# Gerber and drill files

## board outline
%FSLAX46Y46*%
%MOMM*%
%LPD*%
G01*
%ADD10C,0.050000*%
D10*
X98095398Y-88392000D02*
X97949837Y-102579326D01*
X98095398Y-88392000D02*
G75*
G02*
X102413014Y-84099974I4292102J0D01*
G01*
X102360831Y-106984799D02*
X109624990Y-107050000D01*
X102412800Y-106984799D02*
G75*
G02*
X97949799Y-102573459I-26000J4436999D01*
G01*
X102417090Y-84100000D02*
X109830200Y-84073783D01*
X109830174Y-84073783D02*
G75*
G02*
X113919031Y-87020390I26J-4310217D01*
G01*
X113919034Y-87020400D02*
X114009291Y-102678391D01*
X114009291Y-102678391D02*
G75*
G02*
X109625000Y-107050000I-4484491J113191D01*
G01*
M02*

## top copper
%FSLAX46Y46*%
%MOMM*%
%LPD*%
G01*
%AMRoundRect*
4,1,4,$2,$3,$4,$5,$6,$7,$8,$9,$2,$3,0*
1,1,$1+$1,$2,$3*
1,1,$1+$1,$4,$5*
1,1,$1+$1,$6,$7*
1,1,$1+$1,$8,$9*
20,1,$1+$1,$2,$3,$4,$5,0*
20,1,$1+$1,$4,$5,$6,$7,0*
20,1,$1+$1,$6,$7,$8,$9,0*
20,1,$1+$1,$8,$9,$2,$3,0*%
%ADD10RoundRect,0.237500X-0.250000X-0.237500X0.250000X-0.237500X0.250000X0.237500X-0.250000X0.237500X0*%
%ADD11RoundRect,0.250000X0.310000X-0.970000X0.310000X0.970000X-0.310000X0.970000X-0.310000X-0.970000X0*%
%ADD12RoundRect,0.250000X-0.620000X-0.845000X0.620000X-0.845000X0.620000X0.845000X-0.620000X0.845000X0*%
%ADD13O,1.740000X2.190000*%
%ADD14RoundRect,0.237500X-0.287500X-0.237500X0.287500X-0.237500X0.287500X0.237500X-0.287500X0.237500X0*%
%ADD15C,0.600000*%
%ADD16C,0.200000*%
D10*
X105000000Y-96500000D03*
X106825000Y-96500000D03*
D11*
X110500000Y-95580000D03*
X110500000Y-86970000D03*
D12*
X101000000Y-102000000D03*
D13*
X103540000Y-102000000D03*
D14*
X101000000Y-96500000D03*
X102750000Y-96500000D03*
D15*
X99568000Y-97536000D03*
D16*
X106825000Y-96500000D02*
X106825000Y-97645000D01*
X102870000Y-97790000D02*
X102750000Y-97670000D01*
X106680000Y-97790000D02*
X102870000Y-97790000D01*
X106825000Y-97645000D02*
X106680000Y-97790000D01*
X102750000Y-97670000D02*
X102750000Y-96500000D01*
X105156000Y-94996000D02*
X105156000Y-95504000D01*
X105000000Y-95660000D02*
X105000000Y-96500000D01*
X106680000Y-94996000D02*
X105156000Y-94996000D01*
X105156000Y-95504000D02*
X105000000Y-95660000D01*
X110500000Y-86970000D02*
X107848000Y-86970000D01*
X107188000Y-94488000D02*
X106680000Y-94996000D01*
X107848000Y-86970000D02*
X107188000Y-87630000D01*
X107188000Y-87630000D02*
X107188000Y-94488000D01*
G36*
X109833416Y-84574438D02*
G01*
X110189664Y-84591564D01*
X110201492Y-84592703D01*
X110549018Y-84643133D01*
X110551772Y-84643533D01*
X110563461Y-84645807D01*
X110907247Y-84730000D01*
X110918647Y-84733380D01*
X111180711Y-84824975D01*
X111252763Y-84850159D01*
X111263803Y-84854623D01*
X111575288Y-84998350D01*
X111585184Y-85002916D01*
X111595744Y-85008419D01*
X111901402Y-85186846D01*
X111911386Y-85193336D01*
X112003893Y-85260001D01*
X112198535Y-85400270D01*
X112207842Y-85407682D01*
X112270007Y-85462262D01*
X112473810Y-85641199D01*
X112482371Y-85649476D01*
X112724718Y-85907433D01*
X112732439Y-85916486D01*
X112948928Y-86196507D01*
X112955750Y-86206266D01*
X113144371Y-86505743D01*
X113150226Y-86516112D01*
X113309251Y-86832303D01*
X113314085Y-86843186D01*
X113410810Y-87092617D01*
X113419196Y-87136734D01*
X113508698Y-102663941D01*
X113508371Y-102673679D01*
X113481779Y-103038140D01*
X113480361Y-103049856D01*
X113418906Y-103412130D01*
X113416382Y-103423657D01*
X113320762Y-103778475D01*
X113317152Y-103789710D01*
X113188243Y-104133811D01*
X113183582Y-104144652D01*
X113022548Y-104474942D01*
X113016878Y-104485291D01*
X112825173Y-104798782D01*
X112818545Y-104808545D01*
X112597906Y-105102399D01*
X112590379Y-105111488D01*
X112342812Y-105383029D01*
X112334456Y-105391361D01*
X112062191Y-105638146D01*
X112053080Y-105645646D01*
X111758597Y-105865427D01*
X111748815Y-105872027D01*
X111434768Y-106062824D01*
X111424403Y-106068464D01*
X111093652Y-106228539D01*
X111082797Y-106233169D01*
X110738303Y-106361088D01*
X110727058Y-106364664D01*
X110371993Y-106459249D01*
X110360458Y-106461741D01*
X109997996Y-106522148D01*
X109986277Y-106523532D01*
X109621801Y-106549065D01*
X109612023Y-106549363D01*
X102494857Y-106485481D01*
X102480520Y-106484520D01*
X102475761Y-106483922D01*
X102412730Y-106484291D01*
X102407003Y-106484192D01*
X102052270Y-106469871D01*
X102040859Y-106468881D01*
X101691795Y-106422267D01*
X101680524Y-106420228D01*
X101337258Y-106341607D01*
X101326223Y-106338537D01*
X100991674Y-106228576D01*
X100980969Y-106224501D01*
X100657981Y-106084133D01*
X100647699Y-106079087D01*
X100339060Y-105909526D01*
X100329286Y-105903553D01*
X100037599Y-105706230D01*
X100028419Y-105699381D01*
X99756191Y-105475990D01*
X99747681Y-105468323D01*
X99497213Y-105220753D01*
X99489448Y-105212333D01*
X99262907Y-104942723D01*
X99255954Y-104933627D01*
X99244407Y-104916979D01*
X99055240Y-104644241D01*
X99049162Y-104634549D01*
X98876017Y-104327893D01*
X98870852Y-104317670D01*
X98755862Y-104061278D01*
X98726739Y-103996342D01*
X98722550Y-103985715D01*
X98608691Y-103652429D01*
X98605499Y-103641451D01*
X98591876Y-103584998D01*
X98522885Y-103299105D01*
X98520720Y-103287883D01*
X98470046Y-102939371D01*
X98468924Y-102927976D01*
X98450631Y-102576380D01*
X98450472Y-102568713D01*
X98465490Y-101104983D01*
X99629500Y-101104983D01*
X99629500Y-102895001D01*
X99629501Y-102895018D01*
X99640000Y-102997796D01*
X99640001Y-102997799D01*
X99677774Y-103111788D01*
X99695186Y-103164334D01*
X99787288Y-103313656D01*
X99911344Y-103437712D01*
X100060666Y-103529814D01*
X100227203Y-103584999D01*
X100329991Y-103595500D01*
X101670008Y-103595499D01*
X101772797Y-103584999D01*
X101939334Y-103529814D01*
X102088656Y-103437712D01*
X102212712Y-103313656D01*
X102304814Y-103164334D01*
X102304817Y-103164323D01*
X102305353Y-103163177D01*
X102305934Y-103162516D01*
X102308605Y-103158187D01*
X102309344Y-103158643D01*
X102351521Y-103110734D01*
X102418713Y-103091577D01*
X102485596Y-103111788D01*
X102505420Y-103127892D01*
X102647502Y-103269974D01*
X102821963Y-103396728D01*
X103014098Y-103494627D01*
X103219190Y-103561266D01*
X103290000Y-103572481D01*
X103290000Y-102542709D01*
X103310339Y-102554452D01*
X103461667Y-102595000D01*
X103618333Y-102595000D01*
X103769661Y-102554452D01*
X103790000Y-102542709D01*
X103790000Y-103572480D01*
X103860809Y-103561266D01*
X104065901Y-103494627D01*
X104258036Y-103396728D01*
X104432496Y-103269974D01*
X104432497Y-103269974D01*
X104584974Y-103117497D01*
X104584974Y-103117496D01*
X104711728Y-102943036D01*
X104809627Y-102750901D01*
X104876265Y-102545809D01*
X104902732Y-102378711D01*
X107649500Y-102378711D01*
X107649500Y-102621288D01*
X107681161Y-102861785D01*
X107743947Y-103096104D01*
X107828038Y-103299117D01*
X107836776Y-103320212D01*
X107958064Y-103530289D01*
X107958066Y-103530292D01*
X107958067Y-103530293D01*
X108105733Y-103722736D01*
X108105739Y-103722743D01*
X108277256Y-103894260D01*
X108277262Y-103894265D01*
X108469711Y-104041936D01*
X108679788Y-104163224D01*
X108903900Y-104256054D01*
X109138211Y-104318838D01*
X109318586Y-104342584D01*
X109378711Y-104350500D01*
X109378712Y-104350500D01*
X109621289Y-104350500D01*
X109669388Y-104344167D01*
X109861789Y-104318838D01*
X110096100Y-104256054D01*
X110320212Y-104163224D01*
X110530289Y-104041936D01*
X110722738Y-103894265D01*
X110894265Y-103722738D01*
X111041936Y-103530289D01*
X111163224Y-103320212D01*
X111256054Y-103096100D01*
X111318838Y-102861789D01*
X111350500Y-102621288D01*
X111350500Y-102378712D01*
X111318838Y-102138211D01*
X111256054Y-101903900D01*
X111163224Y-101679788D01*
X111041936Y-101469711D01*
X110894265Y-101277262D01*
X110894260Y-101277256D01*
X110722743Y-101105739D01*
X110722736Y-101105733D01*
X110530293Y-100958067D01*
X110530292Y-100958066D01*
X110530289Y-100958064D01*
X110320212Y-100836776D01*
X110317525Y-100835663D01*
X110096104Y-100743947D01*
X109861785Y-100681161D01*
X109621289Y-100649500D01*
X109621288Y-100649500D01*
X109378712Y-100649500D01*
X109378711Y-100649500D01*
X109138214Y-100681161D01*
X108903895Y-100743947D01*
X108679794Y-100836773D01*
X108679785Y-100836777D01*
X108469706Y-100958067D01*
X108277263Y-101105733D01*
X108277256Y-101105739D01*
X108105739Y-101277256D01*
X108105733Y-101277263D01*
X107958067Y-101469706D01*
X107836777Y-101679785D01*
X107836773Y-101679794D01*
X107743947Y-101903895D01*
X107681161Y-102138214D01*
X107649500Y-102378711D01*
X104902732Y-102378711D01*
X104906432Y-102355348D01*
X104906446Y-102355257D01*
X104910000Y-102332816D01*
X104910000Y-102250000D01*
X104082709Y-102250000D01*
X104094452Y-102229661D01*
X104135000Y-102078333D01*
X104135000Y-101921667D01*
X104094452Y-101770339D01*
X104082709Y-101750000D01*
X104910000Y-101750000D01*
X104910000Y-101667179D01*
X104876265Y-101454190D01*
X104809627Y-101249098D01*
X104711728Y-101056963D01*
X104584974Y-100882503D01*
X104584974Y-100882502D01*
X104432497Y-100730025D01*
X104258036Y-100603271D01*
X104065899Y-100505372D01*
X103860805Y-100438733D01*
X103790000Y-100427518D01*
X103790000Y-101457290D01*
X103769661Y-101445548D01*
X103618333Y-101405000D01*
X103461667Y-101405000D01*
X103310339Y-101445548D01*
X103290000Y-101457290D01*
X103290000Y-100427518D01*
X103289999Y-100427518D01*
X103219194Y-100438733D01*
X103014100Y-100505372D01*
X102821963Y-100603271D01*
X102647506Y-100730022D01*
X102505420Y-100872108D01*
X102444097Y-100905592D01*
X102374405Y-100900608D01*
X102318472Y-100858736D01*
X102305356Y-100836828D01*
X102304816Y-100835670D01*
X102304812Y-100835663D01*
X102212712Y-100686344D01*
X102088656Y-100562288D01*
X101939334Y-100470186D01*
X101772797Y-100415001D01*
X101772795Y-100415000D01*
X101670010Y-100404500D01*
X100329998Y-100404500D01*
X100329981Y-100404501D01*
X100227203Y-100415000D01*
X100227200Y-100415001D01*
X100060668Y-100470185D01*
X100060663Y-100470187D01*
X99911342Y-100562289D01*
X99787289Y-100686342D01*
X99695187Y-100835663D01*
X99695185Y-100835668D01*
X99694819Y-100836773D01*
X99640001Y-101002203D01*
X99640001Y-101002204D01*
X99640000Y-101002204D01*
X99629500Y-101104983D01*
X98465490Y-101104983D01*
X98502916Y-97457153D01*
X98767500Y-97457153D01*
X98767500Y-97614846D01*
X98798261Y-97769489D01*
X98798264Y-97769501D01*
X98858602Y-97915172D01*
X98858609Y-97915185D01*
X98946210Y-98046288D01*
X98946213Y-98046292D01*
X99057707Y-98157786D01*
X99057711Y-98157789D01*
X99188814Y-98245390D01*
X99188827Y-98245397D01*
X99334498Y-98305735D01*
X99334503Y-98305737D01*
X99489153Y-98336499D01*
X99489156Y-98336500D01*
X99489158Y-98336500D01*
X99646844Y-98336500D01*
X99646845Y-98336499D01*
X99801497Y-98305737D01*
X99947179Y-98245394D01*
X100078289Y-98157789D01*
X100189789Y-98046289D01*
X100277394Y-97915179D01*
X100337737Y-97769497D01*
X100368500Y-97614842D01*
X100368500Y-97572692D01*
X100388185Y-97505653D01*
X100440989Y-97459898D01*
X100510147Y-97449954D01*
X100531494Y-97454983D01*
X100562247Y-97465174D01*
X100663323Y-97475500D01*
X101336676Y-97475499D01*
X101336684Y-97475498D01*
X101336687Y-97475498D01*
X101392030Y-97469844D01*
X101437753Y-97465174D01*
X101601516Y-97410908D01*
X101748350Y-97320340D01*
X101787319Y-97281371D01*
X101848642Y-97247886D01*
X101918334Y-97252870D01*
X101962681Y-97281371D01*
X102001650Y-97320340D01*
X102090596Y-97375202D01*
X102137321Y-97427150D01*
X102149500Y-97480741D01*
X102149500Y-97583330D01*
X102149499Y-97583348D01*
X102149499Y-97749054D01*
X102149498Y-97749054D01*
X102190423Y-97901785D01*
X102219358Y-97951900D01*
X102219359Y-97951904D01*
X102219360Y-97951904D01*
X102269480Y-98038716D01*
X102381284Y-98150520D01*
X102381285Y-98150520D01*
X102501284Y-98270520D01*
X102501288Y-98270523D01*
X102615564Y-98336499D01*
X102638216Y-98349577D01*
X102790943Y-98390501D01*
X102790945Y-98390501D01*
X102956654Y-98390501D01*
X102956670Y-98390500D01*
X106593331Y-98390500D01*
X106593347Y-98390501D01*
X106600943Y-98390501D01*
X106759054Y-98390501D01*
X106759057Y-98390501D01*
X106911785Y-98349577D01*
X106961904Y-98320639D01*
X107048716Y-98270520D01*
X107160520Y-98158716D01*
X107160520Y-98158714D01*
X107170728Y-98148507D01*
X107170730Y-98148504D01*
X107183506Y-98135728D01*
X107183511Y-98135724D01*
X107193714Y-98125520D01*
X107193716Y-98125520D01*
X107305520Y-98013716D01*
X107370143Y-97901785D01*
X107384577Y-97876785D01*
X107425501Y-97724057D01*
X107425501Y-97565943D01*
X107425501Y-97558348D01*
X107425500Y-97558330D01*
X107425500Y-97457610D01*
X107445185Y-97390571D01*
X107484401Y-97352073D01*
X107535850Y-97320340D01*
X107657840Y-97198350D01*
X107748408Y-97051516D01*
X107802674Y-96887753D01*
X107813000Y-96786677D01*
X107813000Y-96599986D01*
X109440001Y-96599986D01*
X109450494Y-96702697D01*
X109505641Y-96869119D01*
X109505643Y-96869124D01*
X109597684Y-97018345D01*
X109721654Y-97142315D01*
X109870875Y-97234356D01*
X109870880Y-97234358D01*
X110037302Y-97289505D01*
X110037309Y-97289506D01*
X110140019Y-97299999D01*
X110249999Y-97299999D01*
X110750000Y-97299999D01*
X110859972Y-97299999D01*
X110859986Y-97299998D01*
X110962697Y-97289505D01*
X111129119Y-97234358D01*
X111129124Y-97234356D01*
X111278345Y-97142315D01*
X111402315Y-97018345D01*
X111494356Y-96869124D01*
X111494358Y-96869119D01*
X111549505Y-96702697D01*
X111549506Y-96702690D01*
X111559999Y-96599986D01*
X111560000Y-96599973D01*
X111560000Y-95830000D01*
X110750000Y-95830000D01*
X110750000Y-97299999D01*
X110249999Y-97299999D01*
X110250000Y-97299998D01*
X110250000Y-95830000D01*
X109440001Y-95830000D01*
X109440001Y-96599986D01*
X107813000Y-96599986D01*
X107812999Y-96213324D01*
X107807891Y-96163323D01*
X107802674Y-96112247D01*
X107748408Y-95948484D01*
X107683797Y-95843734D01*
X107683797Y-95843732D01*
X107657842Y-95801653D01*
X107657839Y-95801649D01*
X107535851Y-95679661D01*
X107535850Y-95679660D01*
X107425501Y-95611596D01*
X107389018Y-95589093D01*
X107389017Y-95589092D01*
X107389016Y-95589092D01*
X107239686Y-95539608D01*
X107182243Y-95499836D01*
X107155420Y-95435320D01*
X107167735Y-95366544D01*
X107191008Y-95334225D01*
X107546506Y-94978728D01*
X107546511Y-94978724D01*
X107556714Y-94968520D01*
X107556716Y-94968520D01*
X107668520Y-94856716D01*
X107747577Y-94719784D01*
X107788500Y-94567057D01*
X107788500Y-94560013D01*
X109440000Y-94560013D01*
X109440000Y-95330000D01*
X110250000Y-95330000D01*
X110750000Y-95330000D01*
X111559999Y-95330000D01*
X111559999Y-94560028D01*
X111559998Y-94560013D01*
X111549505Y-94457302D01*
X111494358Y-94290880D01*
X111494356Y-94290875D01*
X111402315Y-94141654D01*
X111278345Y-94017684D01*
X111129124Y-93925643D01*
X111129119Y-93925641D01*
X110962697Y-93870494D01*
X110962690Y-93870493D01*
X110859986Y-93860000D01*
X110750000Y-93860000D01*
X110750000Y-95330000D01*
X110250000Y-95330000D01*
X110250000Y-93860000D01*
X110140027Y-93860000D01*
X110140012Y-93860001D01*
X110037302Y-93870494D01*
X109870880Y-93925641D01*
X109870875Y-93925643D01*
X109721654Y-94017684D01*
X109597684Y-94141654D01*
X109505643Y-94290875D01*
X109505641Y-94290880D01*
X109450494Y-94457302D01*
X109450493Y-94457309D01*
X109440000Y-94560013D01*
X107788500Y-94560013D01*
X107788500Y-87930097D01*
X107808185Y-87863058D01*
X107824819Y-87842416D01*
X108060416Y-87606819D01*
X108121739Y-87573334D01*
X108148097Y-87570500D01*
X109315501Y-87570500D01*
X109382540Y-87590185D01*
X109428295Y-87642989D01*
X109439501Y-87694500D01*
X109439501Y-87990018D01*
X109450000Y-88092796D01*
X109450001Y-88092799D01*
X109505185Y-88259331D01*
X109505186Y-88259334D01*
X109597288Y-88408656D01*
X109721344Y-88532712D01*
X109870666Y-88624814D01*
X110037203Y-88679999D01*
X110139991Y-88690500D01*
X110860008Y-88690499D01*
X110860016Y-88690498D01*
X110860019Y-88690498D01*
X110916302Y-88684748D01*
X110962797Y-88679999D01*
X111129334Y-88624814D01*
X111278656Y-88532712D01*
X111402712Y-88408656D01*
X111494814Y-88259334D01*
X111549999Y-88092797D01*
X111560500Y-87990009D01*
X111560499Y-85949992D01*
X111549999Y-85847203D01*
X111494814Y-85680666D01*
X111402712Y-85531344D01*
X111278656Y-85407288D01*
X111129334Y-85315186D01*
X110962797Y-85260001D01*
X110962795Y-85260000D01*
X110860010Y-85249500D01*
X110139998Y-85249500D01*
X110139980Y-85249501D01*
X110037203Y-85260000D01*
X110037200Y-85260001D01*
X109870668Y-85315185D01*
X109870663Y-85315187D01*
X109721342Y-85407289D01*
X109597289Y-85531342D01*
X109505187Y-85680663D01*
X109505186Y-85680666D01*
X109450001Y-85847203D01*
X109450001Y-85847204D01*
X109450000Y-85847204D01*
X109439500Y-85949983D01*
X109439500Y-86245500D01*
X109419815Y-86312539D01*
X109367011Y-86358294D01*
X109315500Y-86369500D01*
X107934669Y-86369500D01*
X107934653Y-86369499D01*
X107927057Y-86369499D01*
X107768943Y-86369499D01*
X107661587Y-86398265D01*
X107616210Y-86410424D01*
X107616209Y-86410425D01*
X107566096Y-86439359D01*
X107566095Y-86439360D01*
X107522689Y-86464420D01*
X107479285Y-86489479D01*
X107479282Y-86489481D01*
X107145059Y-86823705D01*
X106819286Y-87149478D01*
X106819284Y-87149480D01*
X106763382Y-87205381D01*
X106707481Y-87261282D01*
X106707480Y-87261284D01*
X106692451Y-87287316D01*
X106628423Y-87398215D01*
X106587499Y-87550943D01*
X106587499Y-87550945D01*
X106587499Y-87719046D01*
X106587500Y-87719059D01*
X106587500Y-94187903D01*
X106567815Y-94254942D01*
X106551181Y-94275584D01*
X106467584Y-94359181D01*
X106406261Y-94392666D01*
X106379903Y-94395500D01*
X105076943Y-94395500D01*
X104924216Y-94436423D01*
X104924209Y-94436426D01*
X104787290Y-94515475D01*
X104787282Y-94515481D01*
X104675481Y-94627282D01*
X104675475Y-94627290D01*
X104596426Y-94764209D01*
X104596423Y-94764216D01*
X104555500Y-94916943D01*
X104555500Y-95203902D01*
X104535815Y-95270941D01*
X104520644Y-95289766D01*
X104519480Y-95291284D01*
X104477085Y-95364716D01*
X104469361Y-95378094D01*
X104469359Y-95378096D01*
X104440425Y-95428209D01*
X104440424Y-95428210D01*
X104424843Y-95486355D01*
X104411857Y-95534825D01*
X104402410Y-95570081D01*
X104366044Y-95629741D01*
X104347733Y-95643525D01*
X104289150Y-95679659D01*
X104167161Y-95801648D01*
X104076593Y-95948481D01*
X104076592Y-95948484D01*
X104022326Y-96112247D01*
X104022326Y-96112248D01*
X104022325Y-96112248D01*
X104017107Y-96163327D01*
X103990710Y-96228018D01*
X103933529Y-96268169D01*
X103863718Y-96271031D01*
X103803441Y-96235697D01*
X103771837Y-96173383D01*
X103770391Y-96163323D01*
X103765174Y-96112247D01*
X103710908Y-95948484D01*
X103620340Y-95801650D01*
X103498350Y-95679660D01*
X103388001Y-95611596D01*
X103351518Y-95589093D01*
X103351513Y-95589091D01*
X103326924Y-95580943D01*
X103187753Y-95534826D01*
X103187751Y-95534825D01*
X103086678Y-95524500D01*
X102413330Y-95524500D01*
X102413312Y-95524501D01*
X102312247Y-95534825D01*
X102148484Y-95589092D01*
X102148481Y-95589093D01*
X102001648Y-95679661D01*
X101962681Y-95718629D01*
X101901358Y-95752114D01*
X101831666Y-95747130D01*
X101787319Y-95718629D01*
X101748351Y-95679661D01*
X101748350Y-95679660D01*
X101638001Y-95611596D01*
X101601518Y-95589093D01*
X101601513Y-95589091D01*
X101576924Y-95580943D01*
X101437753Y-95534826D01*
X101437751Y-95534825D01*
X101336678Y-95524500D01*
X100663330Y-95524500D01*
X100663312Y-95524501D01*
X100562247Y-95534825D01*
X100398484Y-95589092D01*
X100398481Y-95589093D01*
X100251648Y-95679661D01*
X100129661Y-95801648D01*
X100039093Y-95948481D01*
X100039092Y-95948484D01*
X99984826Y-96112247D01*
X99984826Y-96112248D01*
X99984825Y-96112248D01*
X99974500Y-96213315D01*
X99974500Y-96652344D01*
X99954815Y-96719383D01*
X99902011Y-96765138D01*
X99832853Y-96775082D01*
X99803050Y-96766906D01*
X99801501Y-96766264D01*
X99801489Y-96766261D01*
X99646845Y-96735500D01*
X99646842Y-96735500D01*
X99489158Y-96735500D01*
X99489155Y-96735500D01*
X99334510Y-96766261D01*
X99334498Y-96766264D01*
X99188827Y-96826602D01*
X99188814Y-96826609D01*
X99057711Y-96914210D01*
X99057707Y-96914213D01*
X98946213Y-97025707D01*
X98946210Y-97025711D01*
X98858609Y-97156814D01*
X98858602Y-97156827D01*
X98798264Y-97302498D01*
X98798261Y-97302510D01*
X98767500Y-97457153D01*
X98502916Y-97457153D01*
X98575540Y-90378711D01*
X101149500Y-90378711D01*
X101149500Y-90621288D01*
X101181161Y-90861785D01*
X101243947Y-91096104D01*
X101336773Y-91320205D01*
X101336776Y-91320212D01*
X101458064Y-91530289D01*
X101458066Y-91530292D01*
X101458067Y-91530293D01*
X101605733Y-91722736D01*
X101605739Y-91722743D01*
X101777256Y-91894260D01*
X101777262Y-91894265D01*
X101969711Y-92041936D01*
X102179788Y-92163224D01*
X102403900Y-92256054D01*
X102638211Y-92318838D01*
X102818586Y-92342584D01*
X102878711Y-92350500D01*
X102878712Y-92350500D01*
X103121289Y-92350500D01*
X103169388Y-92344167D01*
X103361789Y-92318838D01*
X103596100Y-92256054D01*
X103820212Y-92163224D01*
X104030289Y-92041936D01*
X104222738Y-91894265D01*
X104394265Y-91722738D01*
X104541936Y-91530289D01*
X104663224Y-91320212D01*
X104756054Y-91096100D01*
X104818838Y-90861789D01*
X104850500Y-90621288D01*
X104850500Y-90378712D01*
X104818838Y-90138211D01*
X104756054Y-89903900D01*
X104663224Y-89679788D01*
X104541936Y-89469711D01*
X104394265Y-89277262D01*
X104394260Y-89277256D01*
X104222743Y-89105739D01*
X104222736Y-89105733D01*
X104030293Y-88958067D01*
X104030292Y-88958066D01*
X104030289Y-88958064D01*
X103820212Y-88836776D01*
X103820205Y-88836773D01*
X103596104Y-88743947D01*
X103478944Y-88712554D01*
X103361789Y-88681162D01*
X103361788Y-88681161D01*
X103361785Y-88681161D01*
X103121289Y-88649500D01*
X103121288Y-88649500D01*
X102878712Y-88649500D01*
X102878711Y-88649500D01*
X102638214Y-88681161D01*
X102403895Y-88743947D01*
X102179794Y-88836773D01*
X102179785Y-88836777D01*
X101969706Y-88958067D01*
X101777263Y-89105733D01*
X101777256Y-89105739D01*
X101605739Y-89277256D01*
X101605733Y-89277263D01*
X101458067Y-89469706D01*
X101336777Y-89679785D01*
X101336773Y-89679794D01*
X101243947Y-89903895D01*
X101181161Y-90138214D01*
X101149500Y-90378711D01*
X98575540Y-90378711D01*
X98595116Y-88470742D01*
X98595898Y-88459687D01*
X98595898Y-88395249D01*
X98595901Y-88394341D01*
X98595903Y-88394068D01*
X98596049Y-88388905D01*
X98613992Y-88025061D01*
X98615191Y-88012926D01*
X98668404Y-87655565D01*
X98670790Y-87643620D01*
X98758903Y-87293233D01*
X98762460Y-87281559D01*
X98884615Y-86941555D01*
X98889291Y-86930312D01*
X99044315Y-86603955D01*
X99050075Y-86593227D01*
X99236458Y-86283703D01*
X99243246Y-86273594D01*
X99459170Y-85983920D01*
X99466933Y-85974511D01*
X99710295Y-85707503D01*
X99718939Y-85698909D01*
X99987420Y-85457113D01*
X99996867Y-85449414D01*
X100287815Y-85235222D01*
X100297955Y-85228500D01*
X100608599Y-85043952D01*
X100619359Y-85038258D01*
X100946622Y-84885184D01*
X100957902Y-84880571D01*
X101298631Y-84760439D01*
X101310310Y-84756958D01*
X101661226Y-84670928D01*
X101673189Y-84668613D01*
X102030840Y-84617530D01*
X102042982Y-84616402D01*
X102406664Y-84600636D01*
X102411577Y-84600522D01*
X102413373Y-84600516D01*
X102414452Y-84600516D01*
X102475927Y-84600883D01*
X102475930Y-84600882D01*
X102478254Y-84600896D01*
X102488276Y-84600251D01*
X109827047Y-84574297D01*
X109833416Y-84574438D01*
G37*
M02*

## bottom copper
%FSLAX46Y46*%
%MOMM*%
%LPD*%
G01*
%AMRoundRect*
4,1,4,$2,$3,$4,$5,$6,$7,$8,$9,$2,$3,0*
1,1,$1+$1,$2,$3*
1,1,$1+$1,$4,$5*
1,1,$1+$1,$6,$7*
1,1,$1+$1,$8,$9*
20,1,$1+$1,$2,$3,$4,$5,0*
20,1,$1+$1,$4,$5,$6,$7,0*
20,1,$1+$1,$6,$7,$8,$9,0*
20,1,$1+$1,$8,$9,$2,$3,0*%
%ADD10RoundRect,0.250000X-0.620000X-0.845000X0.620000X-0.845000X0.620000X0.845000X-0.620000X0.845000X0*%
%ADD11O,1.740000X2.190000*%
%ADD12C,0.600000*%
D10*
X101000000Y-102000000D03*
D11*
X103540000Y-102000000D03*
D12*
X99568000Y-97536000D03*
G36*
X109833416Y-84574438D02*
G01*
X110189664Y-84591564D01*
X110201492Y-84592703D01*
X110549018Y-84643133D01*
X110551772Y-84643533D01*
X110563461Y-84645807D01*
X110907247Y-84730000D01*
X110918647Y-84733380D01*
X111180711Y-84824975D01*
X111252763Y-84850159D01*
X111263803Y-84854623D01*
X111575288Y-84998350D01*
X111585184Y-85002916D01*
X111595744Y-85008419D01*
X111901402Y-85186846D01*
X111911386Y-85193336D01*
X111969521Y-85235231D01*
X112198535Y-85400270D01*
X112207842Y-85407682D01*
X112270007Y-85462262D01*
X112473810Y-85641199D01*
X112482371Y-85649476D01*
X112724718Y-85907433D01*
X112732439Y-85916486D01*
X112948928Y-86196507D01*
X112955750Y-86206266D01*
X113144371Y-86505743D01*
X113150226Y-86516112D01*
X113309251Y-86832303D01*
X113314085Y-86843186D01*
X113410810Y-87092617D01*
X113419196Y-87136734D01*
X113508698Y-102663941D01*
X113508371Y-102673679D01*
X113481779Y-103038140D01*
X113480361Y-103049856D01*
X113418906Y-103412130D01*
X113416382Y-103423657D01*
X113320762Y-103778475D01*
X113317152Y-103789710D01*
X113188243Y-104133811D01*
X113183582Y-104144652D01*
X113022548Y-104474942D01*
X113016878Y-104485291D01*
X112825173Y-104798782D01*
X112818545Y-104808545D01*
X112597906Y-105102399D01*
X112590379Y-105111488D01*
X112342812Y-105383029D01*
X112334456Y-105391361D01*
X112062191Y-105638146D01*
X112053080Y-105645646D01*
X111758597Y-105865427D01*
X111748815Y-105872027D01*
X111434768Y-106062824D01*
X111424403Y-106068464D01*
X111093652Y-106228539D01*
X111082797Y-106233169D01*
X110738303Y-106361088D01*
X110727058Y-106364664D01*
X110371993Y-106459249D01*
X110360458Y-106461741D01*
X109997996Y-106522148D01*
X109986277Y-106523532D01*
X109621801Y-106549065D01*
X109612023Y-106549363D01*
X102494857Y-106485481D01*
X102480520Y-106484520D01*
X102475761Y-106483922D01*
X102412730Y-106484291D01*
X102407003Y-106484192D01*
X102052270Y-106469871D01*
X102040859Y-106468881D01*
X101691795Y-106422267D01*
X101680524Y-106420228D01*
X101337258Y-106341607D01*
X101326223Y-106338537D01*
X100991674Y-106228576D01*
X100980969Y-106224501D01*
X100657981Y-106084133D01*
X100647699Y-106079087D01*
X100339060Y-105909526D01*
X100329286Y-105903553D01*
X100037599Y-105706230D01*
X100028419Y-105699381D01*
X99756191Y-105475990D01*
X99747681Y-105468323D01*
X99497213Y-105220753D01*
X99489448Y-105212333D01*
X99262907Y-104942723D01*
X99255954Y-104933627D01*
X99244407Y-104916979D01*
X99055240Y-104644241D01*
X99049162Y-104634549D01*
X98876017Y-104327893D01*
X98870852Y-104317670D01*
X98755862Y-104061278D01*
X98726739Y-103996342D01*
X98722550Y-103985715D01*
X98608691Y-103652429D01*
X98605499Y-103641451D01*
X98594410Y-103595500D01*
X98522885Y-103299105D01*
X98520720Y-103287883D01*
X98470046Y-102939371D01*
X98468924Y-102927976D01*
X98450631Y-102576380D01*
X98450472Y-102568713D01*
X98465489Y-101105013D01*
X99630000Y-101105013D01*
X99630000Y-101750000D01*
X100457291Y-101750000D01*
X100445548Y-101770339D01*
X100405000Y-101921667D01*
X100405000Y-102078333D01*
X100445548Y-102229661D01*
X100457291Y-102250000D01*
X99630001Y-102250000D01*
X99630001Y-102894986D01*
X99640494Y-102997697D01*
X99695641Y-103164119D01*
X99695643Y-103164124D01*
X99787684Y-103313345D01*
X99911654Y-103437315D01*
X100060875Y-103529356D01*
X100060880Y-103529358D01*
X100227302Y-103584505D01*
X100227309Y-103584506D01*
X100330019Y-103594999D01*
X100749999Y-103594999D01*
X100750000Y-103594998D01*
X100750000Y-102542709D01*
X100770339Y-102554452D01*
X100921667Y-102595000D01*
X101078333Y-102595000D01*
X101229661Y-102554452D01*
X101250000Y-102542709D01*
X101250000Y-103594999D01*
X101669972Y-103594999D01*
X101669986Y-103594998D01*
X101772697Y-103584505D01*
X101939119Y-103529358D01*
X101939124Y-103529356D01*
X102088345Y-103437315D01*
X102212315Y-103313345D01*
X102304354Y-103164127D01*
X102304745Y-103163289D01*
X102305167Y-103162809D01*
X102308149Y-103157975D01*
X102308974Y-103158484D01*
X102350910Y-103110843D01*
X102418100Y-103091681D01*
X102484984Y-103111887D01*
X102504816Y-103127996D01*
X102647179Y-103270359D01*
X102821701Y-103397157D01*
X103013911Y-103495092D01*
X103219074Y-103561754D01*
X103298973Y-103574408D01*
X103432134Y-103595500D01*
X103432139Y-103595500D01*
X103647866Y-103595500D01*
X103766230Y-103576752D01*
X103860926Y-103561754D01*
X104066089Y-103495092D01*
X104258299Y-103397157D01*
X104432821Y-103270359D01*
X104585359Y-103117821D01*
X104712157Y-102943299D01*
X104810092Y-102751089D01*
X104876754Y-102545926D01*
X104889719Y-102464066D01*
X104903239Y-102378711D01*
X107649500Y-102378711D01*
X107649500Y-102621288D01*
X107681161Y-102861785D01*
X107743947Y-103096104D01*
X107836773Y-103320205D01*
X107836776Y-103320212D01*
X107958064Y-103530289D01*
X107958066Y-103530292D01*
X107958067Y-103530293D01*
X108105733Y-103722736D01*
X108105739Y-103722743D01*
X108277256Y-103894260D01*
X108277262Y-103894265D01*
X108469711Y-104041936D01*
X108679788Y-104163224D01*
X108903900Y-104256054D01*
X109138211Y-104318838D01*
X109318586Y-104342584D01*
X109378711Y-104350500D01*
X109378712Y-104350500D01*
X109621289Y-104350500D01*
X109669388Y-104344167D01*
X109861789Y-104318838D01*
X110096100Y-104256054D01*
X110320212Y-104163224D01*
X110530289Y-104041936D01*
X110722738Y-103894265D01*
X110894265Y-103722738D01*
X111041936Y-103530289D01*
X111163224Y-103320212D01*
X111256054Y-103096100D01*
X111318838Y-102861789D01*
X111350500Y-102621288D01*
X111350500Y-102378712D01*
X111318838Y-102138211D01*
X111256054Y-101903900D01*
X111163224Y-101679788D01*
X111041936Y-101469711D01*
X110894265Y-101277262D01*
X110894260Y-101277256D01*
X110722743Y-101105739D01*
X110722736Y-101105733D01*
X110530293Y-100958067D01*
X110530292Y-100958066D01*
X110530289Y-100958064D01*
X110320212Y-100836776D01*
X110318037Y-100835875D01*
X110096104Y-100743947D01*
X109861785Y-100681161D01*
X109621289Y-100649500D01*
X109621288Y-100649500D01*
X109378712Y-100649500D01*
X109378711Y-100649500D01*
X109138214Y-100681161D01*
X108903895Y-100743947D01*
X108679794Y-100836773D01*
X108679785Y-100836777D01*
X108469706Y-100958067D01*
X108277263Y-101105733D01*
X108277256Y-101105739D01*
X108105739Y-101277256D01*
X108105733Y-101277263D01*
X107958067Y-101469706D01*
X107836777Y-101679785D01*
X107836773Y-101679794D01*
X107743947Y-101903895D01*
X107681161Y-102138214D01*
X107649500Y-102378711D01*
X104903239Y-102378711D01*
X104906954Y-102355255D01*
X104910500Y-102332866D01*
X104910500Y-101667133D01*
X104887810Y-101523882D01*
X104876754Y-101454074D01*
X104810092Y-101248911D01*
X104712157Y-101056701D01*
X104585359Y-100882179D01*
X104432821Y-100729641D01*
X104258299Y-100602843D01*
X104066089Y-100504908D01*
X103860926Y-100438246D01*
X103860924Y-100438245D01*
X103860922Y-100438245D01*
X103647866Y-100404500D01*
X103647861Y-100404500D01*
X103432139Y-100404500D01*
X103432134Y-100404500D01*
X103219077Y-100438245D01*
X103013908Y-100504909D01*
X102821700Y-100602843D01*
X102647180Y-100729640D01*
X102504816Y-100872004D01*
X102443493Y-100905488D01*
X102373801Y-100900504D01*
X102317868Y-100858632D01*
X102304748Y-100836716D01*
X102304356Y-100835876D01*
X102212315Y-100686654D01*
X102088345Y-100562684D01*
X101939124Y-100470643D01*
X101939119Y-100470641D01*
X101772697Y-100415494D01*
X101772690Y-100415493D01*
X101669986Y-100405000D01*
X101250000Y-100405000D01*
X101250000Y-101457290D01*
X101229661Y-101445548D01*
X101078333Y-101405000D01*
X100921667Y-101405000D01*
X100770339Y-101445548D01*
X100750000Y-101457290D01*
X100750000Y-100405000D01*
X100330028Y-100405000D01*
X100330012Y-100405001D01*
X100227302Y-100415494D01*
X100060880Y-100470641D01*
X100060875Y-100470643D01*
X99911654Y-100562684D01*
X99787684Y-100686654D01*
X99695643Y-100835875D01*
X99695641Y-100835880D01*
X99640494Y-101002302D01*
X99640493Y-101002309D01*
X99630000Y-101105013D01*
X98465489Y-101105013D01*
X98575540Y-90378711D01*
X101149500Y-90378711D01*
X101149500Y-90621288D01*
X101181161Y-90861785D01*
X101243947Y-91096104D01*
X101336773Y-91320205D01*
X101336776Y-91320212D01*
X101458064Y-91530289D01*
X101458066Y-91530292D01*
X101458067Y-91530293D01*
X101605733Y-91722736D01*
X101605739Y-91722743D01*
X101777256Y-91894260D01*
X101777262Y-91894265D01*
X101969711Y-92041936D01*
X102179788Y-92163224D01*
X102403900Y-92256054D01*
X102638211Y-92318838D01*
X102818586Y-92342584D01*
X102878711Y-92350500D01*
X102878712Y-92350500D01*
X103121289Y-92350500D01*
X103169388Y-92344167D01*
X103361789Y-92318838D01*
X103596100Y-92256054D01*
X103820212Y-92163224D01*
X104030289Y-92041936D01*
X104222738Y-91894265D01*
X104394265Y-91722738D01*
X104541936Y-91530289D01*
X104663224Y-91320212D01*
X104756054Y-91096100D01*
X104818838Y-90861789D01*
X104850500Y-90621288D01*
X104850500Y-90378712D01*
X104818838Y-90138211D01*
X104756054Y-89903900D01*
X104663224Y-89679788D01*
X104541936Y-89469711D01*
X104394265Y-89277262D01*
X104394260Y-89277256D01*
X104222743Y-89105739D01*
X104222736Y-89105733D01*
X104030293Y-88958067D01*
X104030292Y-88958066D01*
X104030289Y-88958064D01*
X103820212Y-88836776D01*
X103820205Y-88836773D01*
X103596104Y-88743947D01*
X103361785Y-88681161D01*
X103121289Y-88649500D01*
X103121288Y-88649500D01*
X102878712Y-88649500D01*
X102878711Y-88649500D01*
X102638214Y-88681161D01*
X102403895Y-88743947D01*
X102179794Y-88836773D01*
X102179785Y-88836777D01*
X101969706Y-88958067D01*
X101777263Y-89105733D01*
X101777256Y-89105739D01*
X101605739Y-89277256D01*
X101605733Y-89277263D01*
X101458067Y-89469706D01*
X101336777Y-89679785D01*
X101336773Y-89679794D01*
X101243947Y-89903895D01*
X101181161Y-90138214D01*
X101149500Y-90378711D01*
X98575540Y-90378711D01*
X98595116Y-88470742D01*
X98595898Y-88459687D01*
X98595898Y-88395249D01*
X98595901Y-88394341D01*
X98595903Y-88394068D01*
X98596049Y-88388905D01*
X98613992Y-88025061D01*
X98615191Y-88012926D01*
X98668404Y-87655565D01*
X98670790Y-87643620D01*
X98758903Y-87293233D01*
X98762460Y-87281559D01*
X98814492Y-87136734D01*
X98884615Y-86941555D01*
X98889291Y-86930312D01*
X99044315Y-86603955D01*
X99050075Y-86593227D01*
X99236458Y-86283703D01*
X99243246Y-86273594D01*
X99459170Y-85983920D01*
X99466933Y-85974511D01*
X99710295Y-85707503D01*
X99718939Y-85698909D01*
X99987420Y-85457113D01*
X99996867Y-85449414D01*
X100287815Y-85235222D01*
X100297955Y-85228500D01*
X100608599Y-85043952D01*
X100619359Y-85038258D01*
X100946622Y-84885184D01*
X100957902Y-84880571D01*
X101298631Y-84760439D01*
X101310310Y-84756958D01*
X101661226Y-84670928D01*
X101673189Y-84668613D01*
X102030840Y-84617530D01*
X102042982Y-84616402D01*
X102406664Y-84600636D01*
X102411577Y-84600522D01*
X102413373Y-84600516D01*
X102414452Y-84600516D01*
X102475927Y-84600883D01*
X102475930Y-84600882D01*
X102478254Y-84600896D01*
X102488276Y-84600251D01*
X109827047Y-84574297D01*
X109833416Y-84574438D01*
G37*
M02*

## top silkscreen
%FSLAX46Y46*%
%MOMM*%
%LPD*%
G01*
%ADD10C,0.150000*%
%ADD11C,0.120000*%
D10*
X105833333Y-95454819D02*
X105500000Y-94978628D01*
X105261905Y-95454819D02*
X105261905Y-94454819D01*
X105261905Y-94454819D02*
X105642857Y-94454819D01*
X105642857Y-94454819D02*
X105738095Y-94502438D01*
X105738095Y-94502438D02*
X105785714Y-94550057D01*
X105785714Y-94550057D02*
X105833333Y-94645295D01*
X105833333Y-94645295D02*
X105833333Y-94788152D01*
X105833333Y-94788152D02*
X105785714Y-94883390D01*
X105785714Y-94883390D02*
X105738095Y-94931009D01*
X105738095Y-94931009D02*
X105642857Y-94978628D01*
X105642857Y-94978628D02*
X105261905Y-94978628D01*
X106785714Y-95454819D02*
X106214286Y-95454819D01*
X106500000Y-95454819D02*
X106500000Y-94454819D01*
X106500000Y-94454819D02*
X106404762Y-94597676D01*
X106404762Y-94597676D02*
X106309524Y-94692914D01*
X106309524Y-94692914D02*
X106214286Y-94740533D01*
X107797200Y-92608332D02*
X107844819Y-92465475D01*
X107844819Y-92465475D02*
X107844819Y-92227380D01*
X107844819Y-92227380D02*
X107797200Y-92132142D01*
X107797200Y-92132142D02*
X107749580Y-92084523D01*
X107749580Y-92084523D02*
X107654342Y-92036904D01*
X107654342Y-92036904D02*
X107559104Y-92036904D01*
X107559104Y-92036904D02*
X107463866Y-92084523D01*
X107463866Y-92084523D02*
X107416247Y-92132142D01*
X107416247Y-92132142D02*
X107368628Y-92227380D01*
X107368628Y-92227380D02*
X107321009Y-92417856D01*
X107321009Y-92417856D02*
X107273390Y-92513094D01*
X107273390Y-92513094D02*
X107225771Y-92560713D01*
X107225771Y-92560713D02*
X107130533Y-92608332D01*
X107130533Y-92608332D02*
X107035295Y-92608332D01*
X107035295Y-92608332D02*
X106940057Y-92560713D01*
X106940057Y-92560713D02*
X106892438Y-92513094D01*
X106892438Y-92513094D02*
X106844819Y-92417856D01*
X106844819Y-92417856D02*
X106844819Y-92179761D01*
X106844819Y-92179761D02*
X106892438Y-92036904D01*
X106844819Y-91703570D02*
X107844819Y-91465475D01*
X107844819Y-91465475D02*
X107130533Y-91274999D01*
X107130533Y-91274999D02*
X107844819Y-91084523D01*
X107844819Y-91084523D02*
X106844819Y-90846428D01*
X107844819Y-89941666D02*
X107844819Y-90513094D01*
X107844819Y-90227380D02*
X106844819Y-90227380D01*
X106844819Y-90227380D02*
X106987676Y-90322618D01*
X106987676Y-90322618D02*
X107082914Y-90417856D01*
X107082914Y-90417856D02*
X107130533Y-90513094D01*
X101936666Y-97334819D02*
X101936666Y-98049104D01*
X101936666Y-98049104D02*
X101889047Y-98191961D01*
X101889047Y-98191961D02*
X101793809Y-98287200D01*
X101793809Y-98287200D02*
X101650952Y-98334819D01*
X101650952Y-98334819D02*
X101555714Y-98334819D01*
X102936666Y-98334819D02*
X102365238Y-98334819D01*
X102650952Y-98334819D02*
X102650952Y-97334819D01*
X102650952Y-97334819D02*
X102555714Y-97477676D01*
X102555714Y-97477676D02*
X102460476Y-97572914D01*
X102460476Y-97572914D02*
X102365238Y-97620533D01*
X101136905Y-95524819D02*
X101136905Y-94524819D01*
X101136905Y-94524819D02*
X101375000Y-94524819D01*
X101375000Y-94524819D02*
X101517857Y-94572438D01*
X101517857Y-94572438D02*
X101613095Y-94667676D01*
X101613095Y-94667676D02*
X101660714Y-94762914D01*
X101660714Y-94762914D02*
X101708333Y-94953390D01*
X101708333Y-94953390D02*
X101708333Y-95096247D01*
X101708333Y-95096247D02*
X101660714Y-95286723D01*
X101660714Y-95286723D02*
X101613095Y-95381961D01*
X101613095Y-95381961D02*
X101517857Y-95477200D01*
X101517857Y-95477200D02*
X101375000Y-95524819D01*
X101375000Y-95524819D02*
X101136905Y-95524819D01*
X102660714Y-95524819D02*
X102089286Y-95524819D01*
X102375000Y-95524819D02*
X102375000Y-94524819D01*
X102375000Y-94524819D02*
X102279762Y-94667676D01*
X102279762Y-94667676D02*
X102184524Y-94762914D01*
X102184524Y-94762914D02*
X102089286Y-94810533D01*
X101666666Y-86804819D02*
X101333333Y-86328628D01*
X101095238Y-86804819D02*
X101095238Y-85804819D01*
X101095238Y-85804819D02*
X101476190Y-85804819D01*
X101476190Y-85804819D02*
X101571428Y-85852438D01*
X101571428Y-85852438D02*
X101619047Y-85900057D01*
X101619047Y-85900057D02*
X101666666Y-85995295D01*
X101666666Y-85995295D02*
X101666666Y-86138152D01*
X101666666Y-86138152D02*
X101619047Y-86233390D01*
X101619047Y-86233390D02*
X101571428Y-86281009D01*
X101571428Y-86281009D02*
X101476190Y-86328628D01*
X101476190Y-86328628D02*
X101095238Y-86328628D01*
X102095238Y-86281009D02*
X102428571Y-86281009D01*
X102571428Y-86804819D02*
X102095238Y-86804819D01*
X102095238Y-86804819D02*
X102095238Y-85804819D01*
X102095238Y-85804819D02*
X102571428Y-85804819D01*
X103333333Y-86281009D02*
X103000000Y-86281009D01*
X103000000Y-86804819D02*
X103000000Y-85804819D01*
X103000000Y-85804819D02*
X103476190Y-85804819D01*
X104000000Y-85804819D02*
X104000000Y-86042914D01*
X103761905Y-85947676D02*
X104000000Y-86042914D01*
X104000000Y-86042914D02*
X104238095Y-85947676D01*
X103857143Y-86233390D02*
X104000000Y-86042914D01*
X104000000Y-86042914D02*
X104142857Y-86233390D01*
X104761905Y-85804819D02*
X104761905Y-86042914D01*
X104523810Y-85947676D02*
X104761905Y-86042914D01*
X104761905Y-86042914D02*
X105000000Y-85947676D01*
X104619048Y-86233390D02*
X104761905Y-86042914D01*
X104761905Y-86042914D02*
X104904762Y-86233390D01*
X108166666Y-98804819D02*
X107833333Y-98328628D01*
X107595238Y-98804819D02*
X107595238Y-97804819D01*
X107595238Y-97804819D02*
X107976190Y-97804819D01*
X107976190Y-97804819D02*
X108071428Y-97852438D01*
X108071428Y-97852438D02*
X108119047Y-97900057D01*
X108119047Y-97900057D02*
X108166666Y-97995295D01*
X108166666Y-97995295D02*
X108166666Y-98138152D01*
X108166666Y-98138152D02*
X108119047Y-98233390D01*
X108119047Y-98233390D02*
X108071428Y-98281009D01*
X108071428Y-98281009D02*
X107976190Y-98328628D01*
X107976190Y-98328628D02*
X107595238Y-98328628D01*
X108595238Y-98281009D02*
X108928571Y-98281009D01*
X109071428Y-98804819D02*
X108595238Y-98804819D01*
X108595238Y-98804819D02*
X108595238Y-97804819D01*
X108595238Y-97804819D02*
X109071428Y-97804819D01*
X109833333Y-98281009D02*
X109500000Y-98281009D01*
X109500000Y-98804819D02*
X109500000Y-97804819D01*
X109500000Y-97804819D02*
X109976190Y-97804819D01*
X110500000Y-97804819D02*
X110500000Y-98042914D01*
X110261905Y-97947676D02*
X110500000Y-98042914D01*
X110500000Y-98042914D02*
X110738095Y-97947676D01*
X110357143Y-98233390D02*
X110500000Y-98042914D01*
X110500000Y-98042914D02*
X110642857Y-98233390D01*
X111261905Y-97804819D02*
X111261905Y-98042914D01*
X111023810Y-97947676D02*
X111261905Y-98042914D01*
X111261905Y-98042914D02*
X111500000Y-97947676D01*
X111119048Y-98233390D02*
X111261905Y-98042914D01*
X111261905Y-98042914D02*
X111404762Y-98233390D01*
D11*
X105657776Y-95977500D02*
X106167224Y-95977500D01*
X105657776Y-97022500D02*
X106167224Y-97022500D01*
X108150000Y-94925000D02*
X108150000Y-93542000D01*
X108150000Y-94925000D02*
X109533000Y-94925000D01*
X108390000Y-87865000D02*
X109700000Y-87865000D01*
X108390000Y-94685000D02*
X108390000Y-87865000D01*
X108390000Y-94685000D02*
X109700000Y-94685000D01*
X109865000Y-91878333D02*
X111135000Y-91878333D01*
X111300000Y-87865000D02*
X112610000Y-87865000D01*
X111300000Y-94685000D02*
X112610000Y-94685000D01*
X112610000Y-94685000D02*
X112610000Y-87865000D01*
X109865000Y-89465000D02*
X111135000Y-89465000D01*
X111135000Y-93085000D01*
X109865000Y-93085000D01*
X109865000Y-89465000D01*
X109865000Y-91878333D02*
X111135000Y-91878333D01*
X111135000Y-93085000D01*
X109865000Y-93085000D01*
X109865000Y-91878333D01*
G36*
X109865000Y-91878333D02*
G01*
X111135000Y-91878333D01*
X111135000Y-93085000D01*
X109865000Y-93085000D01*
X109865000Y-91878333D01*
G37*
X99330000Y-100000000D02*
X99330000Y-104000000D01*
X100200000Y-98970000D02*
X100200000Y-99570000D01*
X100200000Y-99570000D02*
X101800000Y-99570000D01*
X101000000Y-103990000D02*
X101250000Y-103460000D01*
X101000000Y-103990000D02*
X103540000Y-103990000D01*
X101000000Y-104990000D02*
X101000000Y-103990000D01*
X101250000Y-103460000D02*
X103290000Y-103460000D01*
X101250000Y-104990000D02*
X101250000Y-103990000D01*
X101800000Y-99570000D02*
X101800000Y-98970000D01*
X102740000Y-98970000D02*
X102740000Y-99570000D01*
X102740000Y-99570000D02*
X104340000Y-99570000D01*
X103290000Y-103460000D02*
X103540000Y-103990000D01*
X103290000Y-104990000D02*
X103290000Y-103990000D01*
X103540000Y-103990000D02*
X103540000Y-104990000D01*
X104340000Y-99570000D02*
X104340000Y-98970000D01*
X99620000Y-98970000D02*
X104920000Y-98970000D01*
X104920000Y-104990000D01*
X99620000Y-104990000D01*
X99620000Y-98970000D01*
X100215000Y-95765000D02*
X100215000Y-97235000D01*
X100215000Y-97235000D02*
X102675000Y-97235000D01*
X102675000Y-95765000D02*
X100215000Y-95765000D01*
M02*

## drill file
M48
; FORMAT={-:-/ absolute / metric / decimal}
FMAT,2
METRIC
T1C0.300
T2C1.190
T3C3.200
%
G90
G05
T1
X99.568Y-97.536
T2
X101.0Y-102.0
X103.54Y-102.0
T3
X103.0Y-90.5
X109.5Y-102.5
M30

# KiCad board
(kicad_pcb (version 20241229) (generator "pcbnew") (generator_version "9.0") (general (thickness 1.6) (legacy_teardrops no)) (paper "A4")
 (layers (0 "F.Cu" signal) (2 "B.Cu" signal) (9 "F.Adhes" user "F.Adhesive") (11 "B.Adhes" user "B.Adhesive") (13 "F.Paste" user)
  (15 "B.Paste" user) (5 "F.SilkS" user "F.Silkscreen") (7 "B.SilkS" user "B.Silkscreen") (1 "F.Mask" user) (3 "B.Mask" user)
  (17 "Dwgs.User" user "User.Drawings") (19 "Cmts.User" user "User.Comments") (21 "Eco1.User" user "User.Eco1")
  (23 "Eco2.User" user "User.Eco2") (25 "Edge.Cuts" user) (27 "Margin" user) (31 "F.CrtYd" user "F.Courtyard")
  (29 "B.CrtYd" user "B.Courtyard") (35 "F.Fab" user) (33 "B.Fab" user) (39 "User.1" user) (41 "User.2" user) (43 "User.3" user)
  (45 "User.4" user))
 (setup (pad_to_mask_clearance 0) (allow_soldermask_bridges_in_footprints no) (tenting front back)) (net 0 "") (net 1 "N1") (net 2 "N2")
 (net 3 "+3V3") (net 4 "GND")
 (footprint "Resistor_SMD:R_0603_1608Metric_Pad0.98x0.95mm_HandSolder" (layer "F.Cu") (at 105.9125 96.5)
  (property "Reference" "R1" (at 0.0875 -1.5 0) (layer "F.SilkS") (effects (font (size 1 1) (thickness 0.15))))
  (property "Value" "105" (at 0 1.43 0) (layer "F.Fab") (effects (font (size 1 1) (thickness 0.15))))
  (fp_line (start -0.254724 -0.5225) (end 0.254724 -0.5225) (stroke (width 0.12) (type solid)) (layer "F.SilkS"))
  (fp_line (start -0.254724 0.5225) (end 0.254724 0.5225) (stroke (width 0.12) (type solid)) (layer "F.SilkS"))
  (pad "1" smd roundrect (at -0.9125 0) (size 0.975 0.95) (layers "F.Cu" "F.Mask" "F.Paste") (roundrect_rratio 0.25) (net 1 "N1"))
  (pad "2" smd roundrect (at 0.9125 0) (size 0.975 0.95) (layers "F.Cu" "F.Mask" "F.Paste") (roundrect_rratio 0.25) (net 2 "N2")))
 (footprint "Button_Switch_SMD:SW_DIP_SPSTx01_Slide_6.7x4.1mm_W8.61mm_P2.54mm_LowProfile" (layer "F.Cu") (at 110.5 91.275 90)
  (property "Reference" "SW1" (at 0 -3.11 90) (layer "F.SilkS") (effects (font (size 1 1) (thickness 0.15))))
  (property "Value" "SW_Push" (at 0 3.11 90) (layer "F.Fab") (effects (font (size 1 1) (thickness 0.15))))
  (fp_line (start -3.65 -2.35) (end -2.267 -2.35) (stroke (width 0.12) (type solid)) (layer "F.SilkS"))
  (fp_line (start -3.65 -2.35) (end -3.65 -0.967) (stroke (width 0.12) (type solid)) (layer "F.SilkS"))
  (fp_line (start 3.41 -2.11) (end 3.41 -0.8) (stroke (width 0.12) (type solid)) (layer "F.SilkS"))
  (fp_line (start -3.41 -2.11) (end 3.41 -2.11) (stroke (width 0.12) (type solid)) (layer "F.SilkS"))
  (fp_line (start -3.41 -2.11) (end -3.41 -0.8) (stroke (width 0.12) (type solid)) (layer "F.SilkS"))
  (fp_line (start -0.603333 -0.635) (end -0.603333 0.635) (stroke (width 0.12) (type solid)) (layer "F.SilkS"))
  (fp_line (start 3.41 0.8) (end 3.41 2.11) (stroke (width 0.12) (type solid)) (layer "F.SilkS"))
  (fp_line (start -3.41 0.8) (end -3.41 2.11) (stroke (width 0.12) (type solid)) (layer "F.SilkS"))
  (fp_line (start -3.41 2.11) (end 3.41 2.11) (stroke (width 0.12) (type solid)) (layer "F.SilkS"))
  (fp_rect (start -1.81 -0.635) (end 1.81 0.635) (stroke (width 0.12) (type solid)) (fill no) (layer "F.SilkS"))
  (fp_rect (start -1.81 -0.635) (end -0.603333 0.635) (stroke (width 0.12) (type solid)) (fill yes) (layer "F.SilkS"))
  (pad "1" smd roundrect (at -4.305 0 90) (size 2.44 1.12) (layers "F.Cu" "F.Mask" "F.Paste") (roundrect_rratio 0.223214) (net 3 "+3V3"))
  (pad "2" smd roundrect (at 4.305 0 90) (size 2.44 1.12) (layers "F.Cu" "F.Mask" "F.Paste") (roundrect_rratio 0.223214) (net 1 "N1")))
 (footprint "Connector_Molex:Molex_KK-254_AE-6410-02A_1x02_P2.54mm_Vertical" (layer "F.Cu") (at 101 102)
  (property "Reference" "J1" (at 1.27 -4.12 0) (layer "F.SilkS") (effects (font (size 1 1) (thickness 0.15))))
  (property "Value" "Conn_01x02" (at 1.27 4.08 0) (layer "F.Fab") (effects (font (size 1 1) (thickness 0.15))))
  (fp_line (start -1.67 -2) (end -1.67 2) (stroke (width 0.12) (type solid)) (layer "F.SilkS"))
  (fp_line (start -0.8 -3.03) (end -0.8 -2.43) (stroke (width 0.12) (type solid)) (layer "F.SilkS"))
  (fp_line (start -0.8 -2.43) (end 0.8 -2.43) (stroke (width 0.12) (type solid)) (layer "F.SilkS"))
  (fp_line (start 0 1.99) (end 0.25 1.46) (stroke (width 0.12) (type solid)) (layer "F.SilkS"))
  (fp_line (start 0 1.99) (end 2.54 1.99) (stroke (width 0.12) (type solid)) (layer "F.SilkS"))
  (fp_line (start 0 2.99) (end 0 1.99) (stroke (width 0.12) (type solid)) (layer "F.SilkS"))
  (fp_line (start 0.25 1.46) (end 2.29 1.46) (stroke (width 0.12) (type solid)) (layer "F.SilkS"))
  (fp_line (start 0.25 2.99) (end 0.25 1.99) (stroke (width 0.12) (type solid)) (layer "F.SilkS"))
  (fp_line (start 0.8 -2.43) (end 0.8 -3.03) (stroke (width 0.12) (type solid)) (layer "F.SilkS"))
  (fp_line (start 1.74 -3.03) (end 1.74 -2.43) (stroke (width 0.12) (type solid)) (layer "F.SilkS"))
  (fp_line (start 1.74 -2.43) (end 3.34 -2.43) (stroke (width 0.12) (type solid)) (layer "F.SilkS"))
  (fp_line (start 2.29 1.46) (end 2.54 1.99) (stroke (width 0.12) (type solid)) (layer "F.SilkS"))
  (fp_line (start 2.29 2.99) (end 2.29 1.99) (stroke (width 0.12) (type solid)) (layer "F.SilkS"))
  (fp_line (start 2.54 1.99) (end 2.54 2.99) (stroke (width 0.12) (type solid)) (layer "F.SilkS"))
  (fp_line (start 3.34 -2.43) (end 3.34 -3.03) (stroke (width 0.12) (type solid)) (layer "F.SilkS"))
  (fp_rect (start -1.38 -3.03) (end 3.92 2.99) (stroke (width 0.12) (type solid)) (fill no) (layer "F.SilkS"))
  (pad "1" thru_hole roundrect (at 0 0) (size 1.74 2.19) (drill 1.19) (layers "*.Cu" "*.Mask") (remove_unused_layers no)
   (roundrect_rratio 0.143678) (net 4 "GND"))
  (pad "2" thru_hole oval (at 2.54 0) (size 1.74 2.19) (drill 1.19) (layers "*.Cu" "*.Mask") (remove_unused_layers no) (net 3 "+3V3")))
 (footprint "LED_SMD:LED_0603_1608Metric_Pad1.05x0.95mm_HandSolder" (layer "F.Cu") (at 101.875 96.5)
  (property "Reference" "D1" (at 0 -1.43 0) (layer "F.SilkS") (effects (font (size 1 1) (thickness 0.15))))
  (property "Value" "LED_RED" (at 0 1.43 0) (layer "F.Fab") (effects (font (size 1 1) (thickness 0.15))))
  (fp_line (start -1.66 -0.735) (end -1.66 0.735) (stroke (width 0.12) (type solid)) (layer "F.SilkS"))
  (fp_line (start -1.66 0.735) (end 0.8 0.735) (stroke (width 0.12) (type solid)) (layer "F.SilkS"))
  (fp_line (start 0.8 -0.735) (end -1.66 -0.735) (stroke (width 0.12) (type solid)) (layer "F.SilkS"))
  (pad "1" smd roundrect (at -0.875 0) (size 1.05 0.95) (layers "F.Cu" "F.Mask" "F.Paste") (roundrect_rratio 0.25) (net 4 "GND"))
  (pad "2" smd roundrect (at 0.875 0) (size 1.05 0.95) (layers "F.Cu" "F.Mask" "F.Paste") (roundrect_rratio 0.25) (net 2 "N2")))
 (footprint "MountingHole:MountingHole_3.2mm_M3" (layer "F.Cu") (at 103 90.5)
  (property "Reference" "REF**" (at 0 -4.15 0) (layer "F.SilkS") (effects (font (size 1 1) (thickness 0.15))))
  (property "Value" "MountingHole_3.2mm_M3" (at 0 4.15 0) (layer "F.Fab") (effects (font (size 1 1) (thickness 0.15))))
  (pad "" np_thru_hole circle (at 0 0) (size 3.2 3.2) (drill 3.2) (layers "*.Cu" "*.Mask")))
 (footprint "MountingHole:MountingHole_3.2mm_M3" (layer "F.Cu") (at 109.5 102.5)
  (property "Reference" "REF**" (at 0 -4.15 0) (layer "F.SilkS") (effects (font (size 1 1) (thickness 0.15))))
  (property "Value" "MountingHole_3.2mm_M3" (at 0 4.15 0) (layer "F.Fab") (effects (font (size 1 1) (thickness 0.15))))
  (pad "" np_thru_hole circle (at 0 0) (size 3.2 3.2) (drill 3.2) (layers "*.Cu" "*.Mask")))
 (gr_line (start 98.095398 88.392) (end 97.949837 102.579326) (stroke (width 0.05) (type default)) (layer "Edge.Cuts"))
 (gr_arc (start 98.095398 88.392) (mid 99.361561 85.348027) (end 102.413014 84.1) (stroke (width 0.05) (type default)) (layer "Edge.Cuts"))
 (gr_line (start 102.360831 106.984799) (end 109.62499 107.05) (stroke (width 0.05) (type default)) (layer "Edge.Cuts"))
 (gr_arc (start 102.4128 106.984799) (mid 99.267653 105.703487) (end 97.949837 102.573459) (stroke (width 0.05) (type default))
  (layer "Edge.Cuts"))
 (gr_line (start 102.41709 84.1) (end 109.8302 84.073783) (stroke (width 0.05) (type default)) (layer "Edge.Cuts"))
 (gr_arc (start 109.830174 84.073783) (mid 112.350147 84.887189) (end 113.919 87.0204) (stroke (width 0.05) (type default))
  (layer "Edge.Cuts"))
 (gr_line (start 113.919034 87.0204) (end 114.009291 102.678391) (stroke (width 0.05) (type default)) (layer "Edge.Cuts"))
 (gr_arc (start 114.009291 102.678391) (mid 112.692226 105.741815) (end 109.625 107.05) (stroke (width 0.05) (type default))
  (layer "Edge.Cuts"))
 (via (at 99.568 97.536) (size 0.6) (drill 0.3) (layers "F.Cu" "B.Cu") (free yes) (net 4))
 (segment (start 106.825 96.5) (end 106.825 97.645) (width 0.2) (layer "F.Cu") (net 2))
 (segment (start 102.87 97.79) (end 102.75 97.67) (width 0.2) (layer "F.Cu") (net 2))
 (segment (start 106.68 97.79) (end 102.87 97.79) (width 0.2) (layer "F.Cu") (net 2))
 (segment (start 106.825 97.645) (end 106.68 97.79) (width 0.2) (layer "F.Cu") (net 2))
 (segment (start 102.75 97.67) (end 102.75 96.5) (width 0.2) (layer "F.Cu") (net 2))
 (segment (start 105.156 94.996) (end 105.156 95.504) (width 0.2) (layer "F.Cu") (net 1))
 (segment (start 105 95.66) (end 105 96.5) (width 0.2) (layer "F.Cu") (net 1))
 (segment (start 106.68 94.996) (end 105.156 94.996) (width 0.2) (layer "F.Cu") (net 1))
 (segment (start 105.156 95.504) (end 105 95.66) (width 0.2) (layer "F.Cu") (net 1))
 (segment (start 110.5 86.97) (end 107.848 86.97) (width 0.2) (layer "F.Cu") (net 1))
 (segment (start 107.188 94.488) (end 106.68 94.996) (width 0.2) (layer "F.Cu") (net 1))
 (segment (start 107.848 86.97) (end 107.188 87.63) (width 0.2) (layer "F.Cu") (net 1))
 (segment (start 107.188 87.63) (end 107.188 94.488) (width 0.2) (layer "F.Cu") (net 1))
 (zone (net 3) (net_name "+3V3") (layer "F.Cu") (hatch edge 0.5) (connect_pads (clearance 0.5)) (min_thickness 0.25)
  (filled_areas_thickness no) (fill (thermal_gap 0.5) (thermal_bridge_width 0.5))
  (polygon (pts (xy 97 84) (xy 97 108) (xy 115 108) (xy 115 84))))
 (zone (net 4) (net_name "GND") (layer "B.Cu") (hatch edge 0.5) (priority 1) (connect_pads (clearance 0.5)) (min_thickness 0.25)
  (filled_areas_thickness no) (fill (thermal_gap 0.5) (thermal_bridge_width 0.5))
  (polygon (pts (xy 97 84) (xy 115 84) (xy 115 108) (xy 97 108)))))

